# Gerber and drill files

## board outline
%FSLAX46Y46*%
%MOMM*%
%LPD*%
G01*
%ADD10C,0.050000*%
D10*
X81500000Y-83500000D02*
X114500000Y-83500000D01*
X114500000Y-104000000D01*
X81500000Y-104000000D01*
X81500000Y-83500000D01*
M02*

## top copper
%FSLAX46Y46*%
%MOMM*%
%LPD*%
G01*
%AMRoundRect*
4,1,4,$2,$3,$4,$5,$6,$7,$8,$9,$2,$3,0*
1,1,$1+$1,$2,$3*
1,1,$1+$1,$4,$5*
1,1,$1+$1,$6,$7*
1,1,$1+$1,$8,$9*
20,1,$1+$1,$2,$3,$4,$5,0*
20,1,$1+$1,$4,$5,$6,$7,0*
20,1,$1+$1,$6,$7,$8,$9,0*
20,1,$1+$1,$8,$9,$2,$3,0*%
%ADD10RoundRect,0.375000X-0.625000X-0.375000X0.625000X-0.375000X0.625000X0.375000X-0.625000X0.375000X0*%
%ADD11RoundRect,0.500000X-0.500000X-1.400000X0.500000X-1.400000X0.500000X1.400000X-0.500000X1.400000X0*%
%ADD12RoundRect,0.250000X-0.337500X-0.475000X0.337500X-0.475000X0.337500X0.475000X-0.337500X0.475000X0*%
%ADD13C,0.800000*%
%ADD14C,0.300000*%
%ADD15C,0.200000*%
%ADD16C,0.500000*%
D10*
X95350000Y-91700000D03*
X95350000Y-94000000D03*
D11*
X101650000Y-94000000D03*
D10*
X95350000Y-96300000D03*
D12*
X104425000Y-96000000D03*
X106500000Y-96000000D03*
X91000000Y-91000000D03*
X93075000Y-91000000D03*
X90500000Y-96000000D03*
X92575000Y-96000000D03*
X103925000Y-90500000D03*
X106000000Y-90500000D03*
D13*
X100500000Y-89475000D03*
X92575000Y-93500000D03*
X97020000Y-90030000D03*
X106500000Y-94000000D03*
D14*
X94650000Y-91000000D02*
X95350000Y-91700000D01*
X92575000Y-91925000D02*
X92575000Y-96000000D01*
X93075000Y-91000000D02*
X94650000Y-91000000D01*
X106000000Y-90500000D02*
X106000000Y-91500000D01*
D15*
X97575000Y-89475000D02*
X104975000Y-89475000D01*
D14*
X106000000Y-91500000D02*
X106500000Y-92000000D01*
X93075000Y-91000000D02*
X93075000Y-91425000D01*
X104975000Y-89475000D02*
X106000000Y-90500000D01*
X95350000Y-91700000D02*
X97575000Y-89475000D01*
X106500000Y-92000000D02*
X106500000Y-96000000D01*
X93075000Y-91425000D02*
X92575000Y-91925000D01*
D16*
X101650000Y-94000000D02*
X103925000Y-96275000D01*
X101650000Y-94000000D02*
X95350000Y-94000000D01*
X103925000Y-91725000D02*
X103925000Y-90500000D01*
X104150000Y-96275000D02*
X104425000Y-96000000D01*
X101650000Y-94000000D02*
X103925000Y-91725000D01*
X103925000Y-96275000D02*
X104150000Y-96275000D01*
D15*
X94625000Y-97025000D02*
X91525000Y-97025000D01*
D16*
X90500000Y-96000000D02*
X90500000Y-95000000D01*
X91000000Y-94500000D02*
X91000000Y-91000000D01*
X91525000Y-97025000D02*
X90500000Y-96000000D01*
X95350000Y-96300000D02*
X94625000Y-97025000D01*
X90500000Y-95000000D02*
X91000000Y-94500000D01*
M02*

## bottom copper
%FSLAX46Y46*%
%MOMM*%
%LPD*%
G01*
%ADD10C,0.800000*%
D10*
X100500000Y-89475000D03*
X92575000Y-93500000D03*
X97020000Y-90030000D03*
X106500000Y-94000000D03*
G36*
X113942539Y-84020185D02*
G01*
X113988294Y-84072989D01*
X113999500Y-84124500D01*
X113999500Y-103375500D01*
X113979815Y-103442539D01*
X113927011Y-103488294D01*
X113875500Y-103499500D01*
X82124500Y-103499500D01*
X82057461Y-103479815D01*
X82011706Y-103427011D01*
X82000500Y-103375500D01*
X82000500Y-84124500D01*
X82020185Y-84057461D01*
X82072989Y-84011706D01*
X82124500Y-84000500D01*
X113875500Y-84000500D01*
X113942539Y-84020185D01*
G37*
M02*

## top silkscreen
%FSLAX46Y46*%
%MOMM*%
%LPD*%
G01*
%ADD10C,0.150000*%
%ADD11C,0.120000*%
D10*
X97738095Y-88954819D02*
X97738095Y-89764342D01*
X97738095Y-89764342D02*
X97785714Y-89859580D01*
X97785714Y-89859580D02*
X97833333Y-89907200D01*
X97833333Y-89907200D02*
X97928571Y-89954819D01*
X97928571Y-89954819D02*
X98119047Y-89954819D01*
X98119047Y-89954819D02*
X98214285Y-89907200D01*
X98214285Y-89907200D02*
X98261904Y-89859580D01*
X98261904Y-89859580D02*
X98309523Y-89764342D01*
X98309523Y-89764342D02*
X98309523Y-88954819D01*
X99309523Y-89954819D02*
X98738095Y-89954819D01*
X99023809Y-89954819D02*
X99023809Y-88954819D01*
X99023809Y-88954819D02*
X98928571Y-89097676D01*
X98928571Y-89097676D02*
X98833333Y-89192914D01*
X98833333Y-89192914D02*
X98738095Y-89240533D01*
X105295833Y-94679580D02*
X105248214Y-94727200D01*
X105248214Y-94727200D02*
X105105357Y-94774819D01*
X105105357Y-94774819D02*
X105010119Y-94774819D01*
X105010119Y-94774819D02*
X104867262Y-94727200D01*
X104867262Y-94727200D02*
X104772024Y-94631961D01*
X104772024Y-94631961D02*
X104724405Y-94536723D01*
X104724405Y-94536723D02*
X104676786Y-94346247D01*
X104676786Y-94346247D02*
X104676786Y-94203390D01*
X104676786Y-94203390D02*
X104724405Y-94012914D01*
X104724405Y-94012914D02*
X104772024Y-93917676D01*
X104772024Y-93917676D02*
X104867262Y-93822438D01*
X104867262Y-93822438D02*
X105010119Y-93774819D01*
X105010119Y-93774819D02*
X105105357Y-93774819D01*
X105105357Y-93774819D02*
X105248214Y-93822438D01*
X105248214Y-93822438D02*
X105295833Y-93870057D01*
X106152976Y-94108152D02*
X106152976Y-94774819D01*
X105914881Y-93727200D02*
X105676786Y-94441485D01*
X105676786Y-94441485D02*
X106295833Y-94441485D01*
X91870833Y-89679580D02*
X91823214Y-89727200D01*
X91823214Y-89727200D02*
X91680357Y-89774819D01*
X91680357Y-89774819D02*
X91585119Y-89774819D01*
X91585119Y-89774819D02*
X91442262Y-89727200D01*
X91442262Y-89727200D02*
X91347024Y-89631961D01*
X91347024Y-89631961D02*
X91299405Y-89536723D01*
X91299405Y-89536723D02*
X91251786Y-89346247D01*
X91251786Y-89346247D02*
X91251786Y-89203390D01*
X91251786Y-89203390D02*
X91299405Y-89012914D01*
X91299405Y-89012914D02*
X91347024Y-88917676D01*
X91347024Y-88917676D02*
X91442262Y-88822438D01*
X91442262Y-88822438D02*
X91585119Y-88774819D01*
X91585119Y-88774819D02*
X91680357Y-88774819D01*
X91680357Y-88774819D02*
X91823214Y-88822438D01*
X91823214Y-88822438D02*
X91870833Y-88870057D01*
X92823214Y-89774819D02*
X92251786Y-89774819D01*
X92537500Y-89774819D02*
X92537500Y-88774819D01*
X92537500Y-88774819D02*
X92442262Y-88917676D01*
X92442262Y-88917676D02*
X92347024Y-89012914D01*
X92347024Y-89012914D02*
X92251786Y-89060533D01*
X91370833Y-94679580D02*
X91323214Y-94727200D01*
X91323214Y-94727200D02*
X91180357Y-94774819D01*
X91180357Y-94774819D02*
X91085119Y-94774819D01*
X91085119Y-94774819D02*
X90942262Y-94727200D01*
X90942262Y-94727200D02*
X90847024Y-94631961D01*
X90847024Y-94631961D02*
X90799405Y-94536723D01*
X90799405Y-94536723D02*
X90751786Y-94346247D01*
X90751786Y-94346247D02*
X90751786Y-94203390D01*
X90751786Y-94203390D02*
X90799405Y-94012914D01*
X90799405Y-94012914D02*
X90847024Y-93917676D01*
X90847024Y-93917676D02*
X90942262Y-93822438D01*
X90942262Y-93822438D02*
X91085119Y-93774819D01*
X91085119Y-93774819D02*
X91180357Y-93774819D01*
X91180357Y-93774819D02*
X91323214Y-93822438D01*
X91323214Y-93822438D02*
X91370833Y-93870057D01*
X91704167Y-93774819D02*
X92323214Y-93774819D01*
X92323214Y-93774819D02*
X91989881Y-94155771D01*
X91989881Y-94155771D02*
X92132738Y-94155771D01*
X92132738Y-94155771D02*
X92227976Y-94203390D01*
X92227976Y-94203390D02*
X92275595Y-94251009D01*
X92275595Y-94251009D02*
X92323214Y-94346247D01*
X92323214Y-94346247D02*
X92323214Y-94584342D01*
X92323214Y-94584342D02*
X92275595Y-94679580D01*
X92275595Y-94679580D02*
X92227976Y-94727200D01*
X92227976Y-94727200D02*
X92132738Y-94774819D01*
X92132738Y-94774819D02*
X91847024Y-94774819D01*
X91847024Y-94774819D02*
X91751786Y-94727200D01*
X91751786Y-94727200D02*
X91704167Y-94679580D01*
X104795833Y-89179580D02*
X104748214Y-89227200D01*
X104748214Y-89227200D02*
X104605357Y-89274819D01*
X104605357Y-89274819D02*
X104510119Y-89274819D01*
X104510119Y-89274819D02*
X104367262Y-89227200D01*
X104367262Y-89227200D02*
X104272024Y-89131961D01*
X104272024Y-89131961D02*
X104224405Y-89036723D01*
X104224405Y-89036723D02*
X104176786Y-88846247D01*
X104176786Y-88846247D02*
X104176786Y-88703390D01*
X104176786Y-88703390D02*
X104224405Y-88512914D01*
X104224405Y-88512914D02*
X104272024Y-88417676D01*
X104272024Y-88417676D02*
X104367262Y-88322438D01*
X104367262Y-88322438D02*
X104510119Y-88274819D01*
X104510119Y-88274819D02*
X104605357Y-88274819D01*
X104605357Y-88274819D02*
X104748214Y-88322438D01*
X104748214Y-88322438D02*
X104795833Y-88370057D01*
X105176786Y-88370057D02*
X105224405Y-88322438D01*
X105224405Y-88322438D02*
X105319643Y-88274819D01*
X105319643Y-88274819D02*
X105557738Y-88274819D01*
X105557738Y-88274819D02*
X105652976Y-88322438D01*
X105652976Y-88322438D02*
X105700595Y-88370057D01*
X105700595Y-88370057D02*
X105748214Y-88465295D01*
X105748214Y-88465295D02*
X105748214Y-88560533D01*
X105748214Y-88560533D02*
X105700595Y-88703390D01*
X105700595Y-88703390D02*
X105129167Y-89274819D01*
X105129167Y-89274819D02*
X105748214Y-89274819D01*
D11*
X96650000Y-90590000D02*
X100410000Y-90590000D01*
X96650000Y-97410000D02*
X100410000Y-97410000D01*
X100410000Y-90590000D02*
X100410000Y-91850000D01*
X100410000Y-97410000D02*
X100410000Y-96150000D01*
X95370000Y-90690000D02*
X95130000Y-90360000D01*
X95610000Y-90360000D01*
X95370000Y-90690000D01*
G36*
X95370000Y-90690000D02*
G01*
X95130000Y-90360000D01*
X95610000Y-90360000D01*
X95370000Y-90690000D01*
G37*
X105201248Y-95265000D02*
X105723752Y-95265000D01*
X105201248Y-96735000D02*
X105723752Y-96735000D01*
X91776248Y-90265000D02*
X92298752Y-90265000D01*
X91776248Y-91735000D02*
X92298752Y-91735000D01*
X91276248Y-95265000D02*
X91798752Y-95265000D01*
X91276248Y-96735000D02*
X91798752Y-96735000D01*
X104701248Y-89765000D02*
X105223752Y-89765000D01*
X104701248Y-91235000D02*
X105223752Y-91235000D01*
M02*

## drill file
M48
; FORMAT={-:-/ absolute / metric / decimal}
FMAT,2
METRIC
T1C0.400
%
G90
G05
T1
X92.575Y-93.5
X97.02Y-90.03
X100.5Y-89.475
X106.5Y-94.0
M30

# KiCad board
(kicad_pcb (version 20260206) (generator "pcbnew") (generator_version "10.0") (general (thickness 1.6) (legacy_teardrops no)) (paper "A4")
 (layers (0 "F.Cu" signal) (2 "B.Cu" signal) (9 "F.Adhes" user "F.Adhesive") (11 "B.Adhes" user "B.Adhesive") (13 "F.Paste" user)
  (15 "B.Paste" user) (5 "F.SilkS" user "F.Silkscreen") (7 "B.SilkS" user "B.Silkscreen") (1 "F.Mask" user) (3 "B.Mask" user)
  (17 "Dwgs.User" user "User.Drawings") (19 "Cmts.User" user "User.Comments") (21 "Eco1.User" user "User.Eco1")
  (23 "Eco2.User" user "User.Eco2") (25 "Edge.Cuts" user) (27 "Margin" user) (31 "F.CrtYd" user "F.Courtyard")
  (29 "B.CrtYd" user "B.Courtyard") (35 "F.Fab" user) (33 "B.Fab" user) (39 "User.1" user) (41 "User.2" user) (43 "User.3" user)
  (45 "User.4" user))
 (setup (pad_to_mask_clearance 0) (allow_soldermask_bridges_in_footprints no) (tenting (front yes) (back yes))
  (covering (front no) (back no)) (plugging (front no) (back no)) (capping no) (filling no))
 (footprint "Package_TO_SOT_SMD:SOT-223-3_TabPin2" (layer "F.Cu") (at 98.5 94)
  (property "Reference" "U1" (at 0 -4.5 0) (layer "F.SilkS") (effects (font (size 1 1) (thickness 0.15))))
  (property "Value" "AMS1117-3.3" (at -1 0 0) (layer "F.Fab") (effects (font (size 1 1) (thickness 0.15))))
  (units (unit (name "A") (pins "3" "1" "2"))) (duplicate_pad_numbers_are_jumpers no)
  (fp_line (start -1.85 -3.41) (end 1.91 -3.41) (stroke (width 0.12) (type solid)) (layer "F.SilkS"))
  (fp_line (start -1.85 3.41) (end 1.91 3.41) (stroke (width 0.12) (type solid)) (layer "F.SilkS"))
  (fp_line (start 1.91 -3.41) (end 1.91 -2.15) (stroke (width 0.12) (type solid)) (layer "F.SilkS"))
  (fp_line (start 1.91 3.41) (end 1.91 2.15) (stroke (width 0.12) (type solid)) (layer "F.SilkS"))
  (fp_poly
   (pts (xy -3.13 -3.31) (xy -3.37 -3.64) (xy -2.89 -3.64) (xy -3.13 -3.31)) (stroke (width 0.12) (type solid)) (fill yes) (layer "F.SilkS"))
  (pad "1" smd roundrect (at -3.15 -2.3) (size 2 1.5) (layers "F.Cu" "F.Mask" "F.Paste") (roundrect_rratio 0.25) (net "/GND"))
  (pad "2" smd roundrect (at -3.15 0) (size 2 1.5) (layers "F.Cu" "F.Mask" "F.Paste") (roundrect_rratio 0.25) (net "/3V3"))
  (pad "2" smd roundrect (at 3.15 0) (size 2 3.8) (layers "F.Cu" "F.Mask" "F.Paste") (roundrect_rratio 0.25) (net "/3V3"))
  (pad "3" smd roundrect (at -3.15 2.3) (size 2 1.5) (layers "F.Cu" "F.Mask" "F.Paste") (roundrect_rratio 0.25) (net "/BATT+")))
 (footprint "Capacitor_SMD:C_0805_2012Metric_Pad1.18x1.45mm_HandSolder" (layer "F.Cu") (at 105.4625 96)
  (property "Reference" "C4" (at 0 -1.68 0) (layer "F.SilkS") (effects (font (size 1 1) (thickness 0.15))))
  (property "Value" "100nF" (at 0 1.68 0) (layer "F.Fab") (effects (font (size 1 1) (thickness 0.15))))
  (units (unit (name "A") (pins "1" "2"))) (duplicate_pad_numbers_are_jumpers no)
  (fp_line (start -0.261252 -0.735) (end 0.261252 -0.735) (stroke (width 0.12) (type solid)) (layer "F.SilkS"))
  (fp_line (start -0.261252 0.735) (end 0.261252 0.735) (stroke (width 0.12) (type solid)) (layer "F.SilkS"))
  (pad "1" smd roundrect (at -1.0375 0) (size 1.175 1.45) (layers "F.Cu" "F.Mask" "F.Paste") (roundrect_rratio 0.212766) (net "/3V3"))
  (pad "2" smd roundrect (at 1.0375 0) (size 1.175 1.45) (layers "F.Cu" "F.Mask" "F.Paste") (roundrect_rratio 0.212766) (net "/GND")))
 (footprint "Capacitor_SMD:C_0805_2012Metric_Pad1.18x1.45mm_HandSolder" (layer "F.Cu") (at 92.0375 91)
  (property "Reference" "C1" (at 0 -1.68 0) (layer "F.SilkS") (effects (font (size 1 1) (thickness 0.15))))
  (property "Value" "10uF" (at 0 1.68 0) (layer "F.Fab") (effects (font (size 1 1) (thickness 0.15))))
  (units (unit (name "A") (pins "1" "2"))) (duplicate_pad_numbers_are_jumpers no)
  (fp_line (start -0.261252 -0.735) (end 0.261252 -0.735) (stroke (width 0.12) (type solid)) (layer "F.SilkS"))
  (fp_line (start -0.261252 0.735) (end 0.261252 0.735) (stroke (width 0.12) (type solid)) (layer "F.SilkS"))
  (pad "1" smd roundrect (at -1.0375 0) (size 1.175 1.45) (layers "F.Cu" "F.Mask" "F.Paste") (roundrect_rratio 0.212766) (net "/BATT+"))
  (pad "2" smd roundrect (at 1.0375 0) (size 1.175 1.45) (layers "F.Cu" "F.Mask" "F.Paste") (roundrect_rratio 0.212766) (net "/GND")))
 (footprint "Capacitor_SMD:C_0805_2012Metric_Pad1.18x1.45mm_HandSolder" (layer "F.Cu") (at 91.5375 96)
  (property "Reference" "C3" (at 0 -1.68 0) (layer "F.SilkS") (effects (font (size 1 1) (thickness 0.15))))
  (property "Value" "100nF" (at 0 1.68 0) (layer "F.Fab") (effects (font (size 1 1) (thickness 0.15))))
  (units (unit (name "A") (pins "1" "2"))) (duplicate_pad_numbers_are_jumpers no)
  (fp_line (start -0.261252 -0.735) (end 0.261252 -0.735) (stroke (width 0.12) (type solid)) (layer "F.SilkS"))
  (fp_line (start -0.261252 0.735) (end 0.261252 0.735) (stroke (width 0.12) (type solid)) (layer "F.SilkS"))
  (pad "1" smd roundrect (at -1.0375 0) (size 1.175 1.45) (layers "F.Cu" "F.Mask" "F.Paste") (roundrect_rratio 0.212766) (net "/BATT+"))
  (pad "2" smd roundrect (at 1.0375 0) (size 1.175 1.45) (layers "F.Cu" "F.Mask" "F.Paste") (roundrect_rratio 0.212766) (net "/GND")))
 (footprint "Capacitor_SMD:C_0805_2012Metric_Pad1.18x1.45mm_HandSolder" (layer "F.Cu") (at 104.9625 90.5)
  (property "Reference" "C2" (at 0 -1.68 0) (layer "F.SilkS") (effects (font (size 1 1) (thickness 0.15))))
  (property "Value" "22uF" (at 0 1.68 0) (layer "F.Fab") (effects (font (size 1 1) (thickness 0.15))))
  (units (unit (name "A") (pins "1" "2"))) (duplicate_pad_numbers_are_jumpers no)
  (fp_line (start -0.261252 -0.735) (end 0.261252 -0.735) (stroke (width 0.12) (type solid)) (layer "F.SilkS"))
  (fp_line (start -0.261252 0.735) (end 0.261252 0.735) (stroke (width 0.12) (type solid)) (layer "F.SilkS"))
  (pad "1" smd roundrect (at -1.0375 0) (size 1.175 1.45) (layers "F.Cu" "F.Mask" "F.Paste") (roundrect_rratio 0.212766) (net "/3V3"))
  (pad "2" smd roundrect (at 1.0375 0) (size 1.175 1.45) (layers "F.Cu" "F.Mask" "F.Paste") (roundrect_rratio 0.212766) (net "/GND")))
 (gr_rect (start 81.5 83.5) (end 114.5 104) (stroke (width 0.05) (type default)) (fill no) (layer "Edge.Cuts"))
 (segment (start 94.65 91) (end 95.35 91.7) (width 0.3) (layer "F.Cu") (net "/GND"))
 (segment (start 92.575 91.925) (end 92.575 96) (width 0.3) (layer "F.Cu") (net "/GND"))
 (segment (start 93.075 91) (end 94.65 91) (width 0.3) (layer "F.Cu") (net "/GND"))
 (segment (start 106 90.5) (end 106 91.5) (width 0.3) (layer "F.Cu") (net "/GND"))
 (segment (start 97.575 89.475) (end 104.975 89.475) (width 0.2) (layer "F.Cu") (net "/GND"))
 (segment (start 106 91.5) (end 106.5 92) (width 0.3) (layer "F.Cu") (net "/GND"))
 (segment (start 93.075 91) (end 93.075 91.425) (width 0.3) (layer "F.Cu") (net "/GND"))
 (segment (start 104.975 89.475) (end 106 90.5) (width 0.3) (layer "F.Cu") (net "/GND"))
 (segment (start 95.35 91.7) (end 97.575 89.475) (width 0.3) (layer "F.Cu") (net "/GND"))
 (segment (start 106.5 92) (end 106.5 96) (width 0.3) (layer "F.Cu") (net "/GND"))
 (segment (start 93.075 91.425) (end 92.575 91.925) (width 0.3) (layer "F.Cu") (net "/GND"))
 (via (at 100.5 89.475) (size 0.8) (drill 0.4) (layers "F.Cu" "B.Cu") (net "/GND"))
 (via (at 92.575 93.5) (size 0.8) (drill 0.4) (layers "F.Cu" "B.Cu") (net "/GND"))
 (via (at 97.02 90.03) (size 0.8) (drill 0.4) (layers "F.Cu" "B.Cu") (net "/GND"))
 (via (at 106.5 94) (size 0.8) (drill 0.4) (layers "F.Cu" "B.Cu") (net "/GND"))
 (segment (start 101.65 94) (end 103.925 96.275) (width 0.5) (layer "F.Cu") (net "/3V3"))
 (segment (start 101.65 94) (end 95.35 94) (width 0.5) (layer "F.Cu") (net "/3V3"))
 (segment (start 103.925 91.725) (end 103.925 90.5) (width 0.5) (layer "F.Cu") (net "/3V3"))
 (segment (start 104.15 96.275) (end 104.425 96) (width 0.5) (layer "F.Cu") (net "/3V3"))
 (segment (start 101.65 94) (end 103.925 91.725) (width 0.5) (layer "F.Cu") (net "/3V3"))
 (segment (start 103.925 96.275) (end 104.15 96.275) (width 0.5) (layer "F.Cu") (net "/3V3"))
 (segment (start 94.625 97.025) (end 91.525 97.025) (width 0.2) (layer "F.Cu") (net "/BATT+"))
 (segment (start 90.5 96) (end 90.5 95) (width 0.5) (layer "F.Cu") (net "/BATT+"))
 (segment (start 91 94.5) (end 91 91) (width 0.5) (layer "F.Cu") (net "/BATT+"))
 (segment (start 91.525 97.025) (end 90.5 96) (width 0.5) (layer "F.Cu") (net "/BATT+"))
 (segment (start 95.35 96.3) (end 94.625 97.025) (width 0.5) (layer "F.Cu") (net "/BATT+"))
 (segment (start 90.5 95) (end 91 94.5) (width 0.5) (layer "F.Cu") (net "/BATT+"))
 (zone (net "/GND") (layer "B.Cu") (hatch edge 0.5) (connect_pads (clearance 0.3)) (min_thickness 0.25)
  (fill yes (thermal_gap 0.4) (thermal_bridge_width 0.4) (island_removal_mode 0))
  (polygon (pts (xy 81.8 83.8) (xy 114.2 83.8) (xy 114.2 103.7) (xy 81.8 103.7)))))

